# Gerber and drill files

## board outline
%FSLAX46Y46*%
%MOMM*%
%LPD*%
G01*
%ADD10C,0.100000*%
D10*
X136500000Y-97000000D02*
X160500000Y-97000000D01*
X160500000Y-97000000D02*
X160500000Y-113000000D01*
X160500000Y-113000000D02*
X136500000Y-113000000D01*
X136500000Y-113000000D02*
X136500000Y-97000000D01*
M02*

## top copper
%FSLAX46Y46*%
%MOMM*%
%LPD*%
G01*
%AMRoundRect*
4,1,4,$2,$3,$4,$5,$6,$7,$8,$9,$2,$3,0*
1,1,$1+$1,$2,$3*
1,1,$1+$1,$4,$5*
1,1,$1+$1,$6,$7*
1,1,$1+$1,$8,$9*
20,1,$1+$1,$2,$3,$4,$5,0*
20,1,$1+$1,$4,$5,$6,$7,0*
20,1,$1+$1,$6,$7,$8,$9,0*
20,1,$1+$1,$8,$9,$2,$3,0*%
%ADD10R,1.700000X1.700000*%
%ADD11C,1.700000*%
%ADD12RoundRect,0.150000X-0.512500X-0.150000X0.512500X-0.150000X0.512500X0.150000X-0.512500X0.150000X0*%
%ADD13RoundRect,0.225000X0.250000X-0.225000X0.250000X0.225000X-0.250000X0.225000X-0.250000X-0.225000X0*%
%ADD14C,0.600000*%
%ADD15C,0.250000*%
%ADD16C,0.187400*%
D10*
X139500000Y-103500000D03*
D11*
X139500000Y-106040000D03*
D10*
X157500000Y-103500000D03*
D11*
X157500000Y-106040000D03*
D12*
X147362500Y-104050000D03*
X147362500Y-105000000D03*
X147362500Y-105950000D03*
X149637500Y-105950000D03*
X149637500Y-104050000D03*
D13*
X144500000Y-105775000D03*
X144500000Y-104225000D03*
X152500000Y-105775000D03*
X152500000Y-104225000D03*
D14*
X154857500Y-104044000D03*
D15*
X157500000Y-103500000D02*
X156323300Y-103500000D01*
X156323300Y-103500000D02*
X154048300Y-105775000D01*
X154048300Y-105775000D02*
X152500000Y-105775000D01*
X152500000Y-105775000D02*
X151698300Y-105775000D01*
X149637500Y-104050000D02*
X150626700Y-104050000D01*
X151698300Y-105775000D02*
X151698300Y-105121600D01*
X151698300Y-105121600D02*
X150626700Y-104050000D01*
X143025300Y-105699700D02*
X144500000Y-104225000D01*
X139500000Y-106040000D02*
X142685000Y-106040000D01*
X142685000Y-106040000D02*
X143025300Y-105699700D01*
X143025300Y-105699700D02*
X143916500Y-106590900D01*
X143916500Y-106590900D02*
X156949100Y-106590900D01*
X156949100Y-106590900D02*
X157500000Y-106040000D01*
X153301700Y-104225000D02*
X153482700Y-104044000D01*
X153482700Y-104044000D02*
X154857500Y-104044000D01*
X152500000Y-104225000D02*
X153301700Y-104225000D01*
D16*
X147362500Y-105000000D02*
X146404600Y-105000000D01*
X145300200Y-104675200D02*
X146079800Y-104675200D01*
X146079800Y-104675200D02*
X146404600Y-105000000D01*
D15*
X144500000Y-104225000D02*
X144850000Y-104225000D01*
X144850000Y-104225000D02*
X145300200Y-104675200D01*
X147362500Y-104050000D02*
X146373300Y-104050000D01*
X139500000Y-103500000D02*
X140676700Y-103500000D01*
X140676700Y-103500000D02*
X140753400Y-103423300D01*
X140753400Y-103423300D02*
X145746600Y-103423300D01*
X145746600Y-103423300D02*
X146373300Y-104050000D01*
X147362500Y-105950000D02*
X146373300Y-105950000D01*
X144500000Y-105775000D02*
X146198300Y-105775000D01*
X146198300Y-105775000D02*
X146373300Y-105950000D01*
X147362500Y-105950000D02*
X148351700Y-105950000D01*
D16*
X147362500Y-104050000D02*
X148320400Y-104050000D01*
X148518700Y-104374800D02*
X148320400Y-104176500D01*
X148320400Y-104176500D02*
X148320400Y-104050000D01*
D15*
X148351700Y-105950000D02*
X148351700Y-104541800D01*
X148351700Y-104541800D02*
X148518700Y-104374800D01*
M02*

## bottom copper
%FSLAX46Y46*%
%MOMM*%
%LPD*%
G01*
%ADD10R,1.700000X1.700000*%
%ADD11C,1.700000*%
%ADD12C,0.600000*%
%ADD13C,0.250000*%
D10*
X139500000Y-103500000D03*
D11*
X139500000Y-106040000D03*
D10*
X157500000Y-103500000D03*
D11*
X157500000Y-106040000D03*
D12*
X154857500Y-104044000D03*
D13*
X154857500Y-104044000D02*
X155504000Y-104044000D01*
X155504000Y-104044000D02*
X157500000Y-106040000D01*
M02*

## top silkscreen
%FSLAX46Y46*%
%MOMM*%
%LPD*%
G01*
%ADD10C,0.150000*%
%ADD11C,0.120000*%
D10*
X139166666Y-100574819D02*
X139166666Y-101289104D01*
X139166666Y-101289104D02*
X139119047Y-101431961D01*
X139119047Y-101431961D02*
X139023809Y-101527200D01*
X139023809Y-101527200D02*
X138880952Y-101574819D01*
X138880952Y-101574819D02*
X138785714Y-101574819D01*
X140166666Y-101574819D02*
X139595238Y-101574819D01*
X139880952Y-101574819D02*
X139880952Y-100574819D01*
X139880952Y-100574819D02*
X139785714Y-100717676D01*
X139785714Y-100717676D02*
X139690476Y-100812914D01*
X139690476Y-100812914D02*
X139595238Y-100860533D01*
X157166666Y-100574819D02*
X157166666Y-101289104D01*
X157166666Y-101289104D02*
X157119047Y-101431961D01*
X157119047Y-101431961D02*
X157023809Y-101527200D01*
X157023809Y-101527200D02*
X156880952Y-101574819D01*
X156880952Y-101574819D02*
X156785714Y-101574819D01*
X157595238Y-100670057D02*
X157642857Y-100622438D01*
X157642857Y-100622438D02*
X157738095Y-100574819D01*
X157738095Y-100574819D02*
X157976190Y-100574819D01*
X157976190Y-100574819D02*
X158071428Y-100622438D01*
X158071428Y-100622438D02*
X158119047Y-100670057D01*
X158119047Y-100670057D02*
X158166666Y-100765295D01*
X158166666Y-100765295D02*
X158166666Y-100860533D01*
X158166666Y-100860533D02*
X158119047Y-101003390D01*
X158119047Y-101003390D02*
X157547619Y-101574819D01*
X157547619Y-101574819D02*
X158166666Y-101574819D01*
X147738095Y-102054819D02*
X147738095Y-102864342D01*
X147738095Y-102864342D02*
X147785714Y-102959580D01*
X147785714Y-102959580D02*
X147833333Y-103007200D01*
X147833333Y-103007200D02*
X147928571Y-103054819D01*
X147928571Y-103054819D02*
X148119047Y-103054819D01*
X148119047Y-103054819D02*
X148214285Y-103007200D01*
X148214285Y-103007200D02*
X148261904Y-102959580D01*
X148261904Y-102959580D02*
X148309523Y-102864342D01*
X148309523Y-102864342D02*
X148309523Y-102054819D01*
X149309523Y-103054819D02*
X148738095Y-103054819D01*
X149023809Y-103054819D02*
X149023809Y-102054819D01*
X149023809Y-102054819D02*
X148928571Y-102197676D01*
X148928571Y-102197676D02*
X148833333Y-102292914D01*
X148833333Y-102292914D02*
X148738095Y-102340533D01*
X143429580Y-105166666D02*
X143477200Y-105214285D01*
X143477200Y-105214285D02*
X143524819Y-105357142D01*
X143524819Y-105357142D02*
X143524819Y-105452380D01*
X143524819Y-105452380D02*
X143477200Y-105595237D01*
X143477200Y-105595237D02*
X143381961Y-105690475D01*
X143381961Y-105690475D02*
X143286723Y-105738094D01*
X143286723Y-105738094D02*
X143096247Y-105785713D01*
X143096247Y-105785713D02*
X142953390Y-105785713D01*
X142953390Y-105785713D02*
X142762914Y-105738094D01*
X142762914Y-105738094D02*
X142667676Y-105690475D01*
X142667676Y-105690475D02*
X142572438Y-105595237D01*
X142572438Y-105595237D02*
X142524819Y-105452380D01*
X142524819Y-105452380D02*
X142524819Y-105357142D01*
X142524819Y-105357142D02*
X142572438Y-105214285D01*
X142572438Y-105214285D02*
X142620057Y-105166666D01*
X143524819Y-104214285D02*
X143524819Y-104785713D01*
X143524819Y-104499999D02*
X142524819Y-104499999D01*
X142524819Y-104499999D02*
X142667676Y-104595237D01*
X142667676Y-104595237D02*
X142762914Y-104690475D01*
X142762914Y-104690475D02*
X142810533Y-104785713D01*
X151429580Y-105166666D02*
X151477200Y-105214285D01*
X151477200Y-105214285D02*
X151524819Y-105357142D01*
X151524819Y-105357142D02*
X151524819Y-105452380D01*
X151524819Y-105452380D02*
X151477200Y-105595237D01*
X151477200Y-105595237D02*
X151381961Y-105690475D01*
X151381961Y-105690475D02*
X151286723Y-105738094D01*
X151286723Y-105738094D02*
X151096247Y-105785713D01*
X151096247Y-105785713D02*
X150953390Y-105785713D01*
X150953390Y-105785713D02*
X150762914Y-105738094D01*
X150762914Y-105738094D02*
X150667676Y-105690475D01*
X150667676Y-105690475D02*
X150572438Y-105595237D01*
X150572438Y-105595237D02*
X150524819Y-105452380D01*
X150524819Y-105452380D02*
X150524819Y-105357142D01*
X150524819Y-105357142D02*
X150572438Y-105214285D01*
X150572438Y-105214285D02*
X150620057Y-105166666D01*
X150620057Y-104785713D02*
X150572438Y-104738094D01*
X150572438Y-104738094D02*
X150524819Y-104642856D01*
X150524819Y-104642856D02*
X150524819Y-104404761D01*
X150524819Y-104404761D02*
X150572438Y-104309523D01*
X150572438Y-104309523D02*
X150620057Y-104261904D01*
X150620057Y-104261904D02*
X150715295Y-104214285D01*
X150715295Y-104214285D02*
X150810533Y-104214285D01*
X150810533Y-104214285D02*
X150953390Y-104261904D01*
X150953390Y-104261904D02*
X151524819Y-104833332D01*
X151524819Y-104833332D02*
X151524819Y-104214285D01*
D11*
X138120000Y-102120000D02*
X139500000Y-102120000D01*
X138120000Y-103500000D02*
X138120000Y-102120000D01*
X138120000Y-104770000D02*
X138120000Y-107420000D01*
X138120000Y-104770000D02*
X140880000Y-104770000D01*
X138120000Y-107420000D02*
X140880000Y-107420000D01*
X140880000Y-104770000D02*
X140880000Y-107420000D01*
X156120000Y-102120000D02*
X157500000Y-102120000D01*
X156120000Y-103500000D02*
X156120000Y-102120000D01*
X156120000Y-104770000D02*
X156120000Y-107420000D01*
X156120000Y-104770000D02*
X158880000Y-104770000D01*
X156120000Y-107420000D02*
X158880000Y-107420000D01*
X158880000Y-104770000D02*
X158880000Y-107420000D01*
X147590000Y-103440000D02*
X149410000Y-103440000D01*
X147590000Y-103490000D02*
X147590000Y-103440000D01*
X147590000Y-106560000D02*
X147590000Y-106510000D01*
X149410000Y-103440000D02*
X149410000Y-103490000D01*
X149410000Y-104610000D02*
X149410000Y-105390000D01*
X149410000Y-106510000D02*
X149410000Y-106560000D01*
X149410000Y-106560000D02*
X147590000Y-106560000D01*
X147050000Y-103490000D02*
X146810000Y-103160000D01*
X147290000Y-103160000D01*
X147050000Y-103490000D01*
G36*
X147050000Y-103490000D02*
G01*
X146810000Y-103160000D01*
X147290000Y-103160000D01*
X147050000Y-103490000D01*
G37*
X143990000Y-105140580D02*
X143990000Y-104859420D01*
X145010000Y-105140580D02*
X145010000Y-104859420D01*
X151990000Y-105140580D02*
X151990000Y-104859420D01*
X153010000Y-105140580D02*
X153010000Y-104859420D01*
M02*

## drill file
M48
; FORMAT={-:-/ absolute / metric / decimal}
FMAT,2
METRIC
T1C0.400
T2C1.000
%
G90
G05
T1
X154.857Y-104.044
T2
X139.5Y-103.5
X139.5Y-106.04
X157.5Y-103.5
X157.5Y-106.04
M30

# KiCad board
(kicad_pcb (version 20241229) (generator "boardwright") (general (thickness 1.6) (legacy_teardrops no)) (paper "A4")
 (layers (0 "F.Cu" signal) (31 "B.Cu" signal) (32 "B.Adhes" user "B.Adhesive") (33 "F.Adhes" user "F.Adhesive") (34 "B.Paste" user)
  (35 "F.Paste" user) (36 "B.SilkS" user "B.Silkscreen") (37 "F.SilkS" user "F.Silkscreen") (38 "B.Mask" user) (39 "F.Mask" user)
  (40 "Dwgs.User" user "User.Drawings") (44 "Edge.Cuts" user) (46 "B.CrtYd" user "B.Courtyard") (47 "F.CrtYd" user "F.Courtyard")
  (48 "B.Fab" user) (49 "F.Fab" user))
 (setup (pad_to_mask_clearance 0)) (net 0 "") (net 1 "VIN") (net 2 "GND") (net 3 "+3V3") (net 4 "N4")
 (gr_line (start 136.5 97) (end 160.5 97) (stroke (width 0.1) (type default)) (layer "Edge.Cuts"))
 (gr_line (start 160.5 97) (end 160.5 113) (stroke (width 0.1) (type default)) (layer "Edge.Cuts"))
 (gr_line (start 160.5 113) (end 136.5 113) (stroke (width 0.1) (type default)) (layer "Edge.Cuts"))
 (gr_line (start 136.5 113) (end 136.5 97) (stroke (width 0.1) (type default)) (layer "Edge.Cuts"))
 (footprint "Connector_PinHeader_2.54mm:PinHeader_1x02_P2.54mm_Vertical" (layer "F.Cu") (at 139.5 103.5)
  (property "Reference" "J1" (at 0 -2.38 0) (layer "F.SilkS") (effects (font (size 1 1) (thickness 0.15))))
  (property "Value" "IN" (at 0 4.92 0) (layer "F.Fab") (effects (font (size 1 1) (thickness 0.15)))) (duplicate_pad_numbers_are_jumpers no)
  (fp_line (start -1.38 -1.38) (end 0 -1.38) (stroke (width 0.12) (type solid)) (layer "F.SilkS"))
  (fp_line (start -1.38 0) (end -1.38 -1.38) (stroke (width 0.12) (type solid)) (layer "F.SilkS"))
  (fp_line (start -1.38 1.27) (end -1.38 3.92) (stroke (width 0.12) (type solid)) (layer "F.SilkS"))
  (fp_line (start -1.38 1.27) (end 1.38 1.27) (stroke (width 0.12) (type solid)) (layer "F.SilkS"))
  (fp_line (start -1.38 3.92) (end 1.38 3.92) (stroke (width 0.12) (type solid)) (layer "F.SilkS"))
  (fp_line (start 1.38 1.27) (end 1.38 3.92) (stroke (width 0.12) (type solid)) (layer "F.SilkS"))
  (pad "1" thru_hole rect (at 0 0) (size 1.7 1.7) (drill 1) (layers "*.Cu" "*.Mask") (remove_unused_layers no) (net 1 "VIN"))
  (pad "2" thru_hole circle (at 0 2.54) (size 1.7 1.7) (drill 1) (layers "*.Cu" "*.Mask") (remove_unused_layers no) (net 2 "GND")))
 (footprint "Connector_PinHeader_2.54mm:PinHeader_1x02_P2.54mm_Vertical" (layer "F.Cu") (at 157.5 103.5)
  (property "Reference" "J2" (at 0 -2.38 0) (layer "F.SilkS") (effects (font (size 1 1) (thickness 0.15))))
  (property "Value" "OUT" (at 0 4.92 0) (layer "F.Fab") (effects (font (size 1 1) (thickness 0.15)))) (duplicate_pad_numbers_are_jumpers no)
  (fp_line (start -1.38 -1.38) (end 0 -1.38) (stroke (width 0.12) (type solid)) (layer "F.SilkS"))
  (fp_line (start -1.38 0) (end -1.38 -1.38) (stroke (width 0.12) (type solid)) (layer "F.SilkS"))
  (fp_line (start -1.38 1.27) (end -1.38 3.92) (stroke (width 0.12) (type solid)) (layer "F.SilkS"))
  (fp_line (start -1.38 1.27) (end 1.38 1.27) (stroke (width 0.12) (type solid)) (layer "F.SilkS"))
  (fp_line (start -1.38 3.92) (end 1.38 3.92) (stroke (width 0.12) (type solid)) (layer "F.SilkS"))
  (fp_line (start 1.38 1.27) (end 1.38 3.92) (stroke (width 0.12) (type solid)) (layer "F.SilkS"))
  (pad "1" thru_hole rect (at 0 0) (size 1.7 1.7) (drill 1) (layers "*.Cu" "*.Mask") (remove_unused_layers no) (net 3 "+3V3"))
  (pad "2" thru_hole circle (at 0 2.54) (size 1.7 1.7) (drill 1) (layers "*.Cu" "*.Mask") (remove_unused_layers no) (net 2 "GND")))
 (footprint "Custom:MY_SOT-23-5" (layer "F.Cu") (at 148.5 105)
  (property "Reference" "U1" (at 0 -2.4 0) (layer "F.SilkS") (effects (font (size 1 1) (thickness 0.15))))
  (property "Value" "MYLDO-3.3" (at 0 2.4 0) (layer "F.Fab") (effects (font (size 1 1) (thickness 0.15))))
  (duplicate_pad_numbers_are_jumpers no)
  (fp_line (start -0.91 -1.56) (end 0.91 -1.56) (stroke (width 0.12) (type solid)) (layer "F.SilkS"))
  (fp_line (start -0.91 -1.51) (end -0.91 -1.56) (stroke (width 0.12) (type solid)) (layer "F.SilkS"))
  (fp_line (start -0.91 1.56) (end -0.91 1.51) (stroke (width 0.12) (type solid)) (layer "F.SilkS"))
  (fp_line (start 0.91 -1.56) (end 0.91 -1.51) (stroke (width 0.12) (type solid)) (layer "F.SilkS"))
  (fp_line (start 0.91 -0.39) (end 0.91 0.39) (stroke (width 0.12) (type solid)) (layer "F.SilkS"))
  (fp_line (start 0.91 1.51) (end 0.91 1.56) (stroke (width 0.12) (type solid)) (layer "F.SilkS"))
  (fp_line (start 0.91 1.56) (end -0.91 1.56) (stroke (width 0.12) (type solid)) (layer "F.SilkS"))
  (fp_poly (pts (xy -1.45 -1.51) (xy -1.69 -1.84) (xy -1.21 -1.84)) (stroke (width 0.12) (type solid)) (fill yes) (layer "F.SilkS"))
  (pad "1" smd roundrect (at -1.1375 -0.95) (size 1.325 0.6) (layers "F.Cu" "F.Mask" "F.Paste") (roundrect_rratio 0.25) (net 1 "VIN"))
  (pad "2" smd roundrect (at -1.1375 0) (size 1.325 0.6) (layers "F.Cu" "F.Mask" "F.Paste") (roundrect_rratio 0.25) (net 2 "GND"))
  (pad "3" smd roundrect (at -1.1375 0.95) (size 1.325 0.6) (layers "F.Cu" "F.Mask" "F.Paste") (roundrect_rratio 0.25) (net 1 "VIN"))
  (pad "4" smd roundrect (at 1.1375 0.95) (size 1.325 0.6) (layers "F.Cu" "F.Mask" "F.Paste") (roundrect_rratio 0.25) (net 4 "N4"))
  (pad "5" smd roundrect (at 1.1375 -0.95) (size 1.325 0.6) (layers "F.Cu" "F.Mask" "F.Paste") (roundrect_rratio 0.25) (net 3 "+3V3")))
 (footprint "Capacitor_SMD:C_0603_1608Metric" (layer "F.Cu") (at 144.5 105 90)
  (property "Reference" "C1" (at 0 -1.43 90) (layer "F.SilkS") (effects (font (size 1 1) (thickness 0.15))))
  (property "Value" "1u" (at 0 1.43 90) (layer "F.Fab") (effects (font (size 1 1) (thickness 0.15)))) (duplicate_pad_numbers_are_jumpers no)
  (fp_line (start -0.14058 -0.51) (end 0.14058 -0.51) (stroke (width 0.12) (type solid)) (layer "F.SilkS"))
  (fp_line (start -0.14058 0.51) (end 0.14058 0.51) (stroke (width 0.12) (type solid)) (layer "F.SilkS"))
  (pad "1" smd roundrect (at -0.775 0 90) (size 0.9 0.95) (layers "F.Cu" "F.Mask" "F.Paste") (roundrect_rratio 0.25) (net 1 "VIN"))
  (pad "2" smd roundrect (at 0.775 0 90) (size 0.9 0.95) (layers "F.Cu" "F.Mask" "F.Paste") (roundrect_rratio 0.25) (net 2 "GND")))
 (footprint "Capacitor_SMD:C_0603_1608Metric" (layer "F.Cu") (at 152.5 105 90)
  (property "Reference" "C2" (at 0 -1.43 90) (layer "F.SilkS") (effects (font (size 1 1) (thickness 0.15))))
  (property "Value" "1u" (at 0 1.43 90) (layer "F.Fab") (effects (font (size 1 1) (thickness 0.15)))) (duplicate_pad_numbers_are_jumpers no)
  (fp_line (start -0.14058 -0.51) (end 0.14058 -0.51) (stroke (width 0.12) (type solid)) (layer "F.SilkS"))
  (fp_line (start -0.14058 0.51) (end 0.14058 0.51) (stroke (width 0.12) (type solid)) (layer "F.SilkS"))
  (pad "1" smd roundrect (at -0.775 0 90) (size 0.9 0.95) (layers "F.Cu" "F.Mask" "F.Paste") (roundrect_rratio 0.25) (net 3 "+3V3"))
  (pad "2" smd roundrect (at 0.775 0 90) (size 0.9 0.95) (layers "F.Cu" "F.Mask" "F.Paste") (roundrect_rratio 0.25) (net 2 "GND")))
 (segment (start 157.5 103.5) (end 156.3233 103.5) (width 0.25) (layer "F.Cu") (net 3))
 (segment (start 156.3233 103.5) (end 154.0483 105.775) (width 0.25) (layer "F.Cu") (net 3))
 (segment (start 154.0483 105.775) (end 152.5 105.775) (width 0.25) (layer "F.Cu") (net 3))
 (segment (start 152.5 105.775) (end 151.6983 105.775) (width 0.25) (layer "F.Cu") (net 3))
 (segment (start 149.6375 104.05) (end 150.6267 104.05) (width 0.25) (layer "F.Cu") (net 3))
 (segment (start 151.6983 105.775) (end 151.6983 105.1216) (width 0.25) (layer "F.Cu") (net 3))
 (segment (start 151.6983 105.1216) (end 150.6267 104.05) (width 0.25) (layer "F.Cu") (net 3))
 (segment (start 143.0253 105.6997) (end 144.5 104.225) (width 0.25) (layer "F.Cu") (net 2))
 (segment (start 139.5 106.04) (end 142.685 106.04) (width 0.25) (layer "F.Cu") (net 2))
 (segment (start 142.685 106.04) (end 143.0253 105.6997) (width 0.25) (layer "F.Cu") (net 2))
 (segment (start 143.0253 105.6997) (end 143.9165 106.5909) (width 0.25) (layer "F.Cu") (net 2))
 (segment (start 143.9165 106.5909) (end 156.9491 106.5909) (width 0.25) (layer "F.Cu") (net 2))
 (segment (start 156.9491 106.5909) (end 157.5 106.04) (width 0.25) (layer "F.Cu") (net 2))
 (segment (start 153.3017 104.225) (end 153.4827 104.044) (width 0.25) (layer "F.Cu") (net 2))
 (segment (start 153.4827 104.044) (end 154.8575 104.044) (width 0.25) (layer "F.Cu") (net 2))
 (segment (start 154.8575 104.044) (end 155.504 104.044) (width 0.25) (layer "B.Cu") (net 2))
 (segment (start 155.504 104.044) (end 157.5 106.04) (width 0.25) (layer "B.Cu") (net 2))
 (segment (start 152.5 104.225) (end 153.3017 104.225) (width 0.25) (layer "F.Cu") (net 2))
 (segment (start 147.3625 105) (end 146.4046 105) (width 0.1874) (layer "F.Cu") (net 2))
 (segment (start 145.3002 104.6752) (end 146.0798 104.6752) (width 0.1874) (layer "F.Cu") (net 2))
 (segment (start 146.0798 104.6752) (end 146.4046 105) (width 0.1874) (layer "F.Cu") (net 2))
 (segment (start 144.5 104.225) (end 144.85 104.225) (width 0.25) (layer "F.Cu") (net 2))
 (segment (start 144.85 104.225) (end 145.3002 104.6752) (width 0.25) (layer "F.Cu") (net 2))
 (segment (start 147.3625 104.05) (end 146.3733 104.05) (width 0.25) (layer "F.Cu") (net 1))
 (segment (start 139.5 103.5) (end 140.6767 103.5) (width 0.25) (layer "F.Cu") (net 1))
 (segment (start 140.6767 103.5) (end 140.7534 103.4233) (width 0.25) (layer "F.Cu") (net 1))
 (segment (start 140.7534 103.4233) (end 145.7466 103.4233) (width 0.25) (layer "F.Cu") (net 1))
 (segment (start 145.7466 103.4233) (end 146.3733 104.05) (width 0.25) (layer "F.Cu") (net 1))
 (segment (start 147.3625 105.95) (end 146.3733 105.95) (width 0.25) (layer "F.Cu") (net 1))
 (segment (start 144.5 105.775) (end 146.1983 105.775) (width 0.25) (layer "F.Cu") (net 1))
 (segment (start 146.1983 105.775) (end 146.3733 105.95) (width 0.25) (layer "F.Cu") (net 1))
 (segment (start 147.3625 105.95) (end 148.3517 105.95) (width 0.25) (layer "F.Cu") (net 1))
 (segment (start 147.3625 104.05) (end 148.3204 104.05) (width 0.1874) (layer "F.Cu") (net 1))
 (segment (start 148.5187 104.3748) (end 148.3204 104.1765) (width 0.1874) (layer "F.Cu") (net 1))
 (segment (start 148.3204 104.1765) (end 148.3204 104.05) (width 0.1874) (layer "F.Cu") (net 1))
 (segment (start 148.3517 105.95) (end 148.3517 104.5418) (width 0.25) (layer "F.Cu") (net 1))
 (segment (start 148.3517 104.5418) (end 148.5187 104.3748) (width 0.25) (layer "F.Cu") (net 1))
 (via (at 154.8575 104.044) (size 0.6) (drill 0.4) (layers "F.Cu" "B.Cu") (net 2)))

